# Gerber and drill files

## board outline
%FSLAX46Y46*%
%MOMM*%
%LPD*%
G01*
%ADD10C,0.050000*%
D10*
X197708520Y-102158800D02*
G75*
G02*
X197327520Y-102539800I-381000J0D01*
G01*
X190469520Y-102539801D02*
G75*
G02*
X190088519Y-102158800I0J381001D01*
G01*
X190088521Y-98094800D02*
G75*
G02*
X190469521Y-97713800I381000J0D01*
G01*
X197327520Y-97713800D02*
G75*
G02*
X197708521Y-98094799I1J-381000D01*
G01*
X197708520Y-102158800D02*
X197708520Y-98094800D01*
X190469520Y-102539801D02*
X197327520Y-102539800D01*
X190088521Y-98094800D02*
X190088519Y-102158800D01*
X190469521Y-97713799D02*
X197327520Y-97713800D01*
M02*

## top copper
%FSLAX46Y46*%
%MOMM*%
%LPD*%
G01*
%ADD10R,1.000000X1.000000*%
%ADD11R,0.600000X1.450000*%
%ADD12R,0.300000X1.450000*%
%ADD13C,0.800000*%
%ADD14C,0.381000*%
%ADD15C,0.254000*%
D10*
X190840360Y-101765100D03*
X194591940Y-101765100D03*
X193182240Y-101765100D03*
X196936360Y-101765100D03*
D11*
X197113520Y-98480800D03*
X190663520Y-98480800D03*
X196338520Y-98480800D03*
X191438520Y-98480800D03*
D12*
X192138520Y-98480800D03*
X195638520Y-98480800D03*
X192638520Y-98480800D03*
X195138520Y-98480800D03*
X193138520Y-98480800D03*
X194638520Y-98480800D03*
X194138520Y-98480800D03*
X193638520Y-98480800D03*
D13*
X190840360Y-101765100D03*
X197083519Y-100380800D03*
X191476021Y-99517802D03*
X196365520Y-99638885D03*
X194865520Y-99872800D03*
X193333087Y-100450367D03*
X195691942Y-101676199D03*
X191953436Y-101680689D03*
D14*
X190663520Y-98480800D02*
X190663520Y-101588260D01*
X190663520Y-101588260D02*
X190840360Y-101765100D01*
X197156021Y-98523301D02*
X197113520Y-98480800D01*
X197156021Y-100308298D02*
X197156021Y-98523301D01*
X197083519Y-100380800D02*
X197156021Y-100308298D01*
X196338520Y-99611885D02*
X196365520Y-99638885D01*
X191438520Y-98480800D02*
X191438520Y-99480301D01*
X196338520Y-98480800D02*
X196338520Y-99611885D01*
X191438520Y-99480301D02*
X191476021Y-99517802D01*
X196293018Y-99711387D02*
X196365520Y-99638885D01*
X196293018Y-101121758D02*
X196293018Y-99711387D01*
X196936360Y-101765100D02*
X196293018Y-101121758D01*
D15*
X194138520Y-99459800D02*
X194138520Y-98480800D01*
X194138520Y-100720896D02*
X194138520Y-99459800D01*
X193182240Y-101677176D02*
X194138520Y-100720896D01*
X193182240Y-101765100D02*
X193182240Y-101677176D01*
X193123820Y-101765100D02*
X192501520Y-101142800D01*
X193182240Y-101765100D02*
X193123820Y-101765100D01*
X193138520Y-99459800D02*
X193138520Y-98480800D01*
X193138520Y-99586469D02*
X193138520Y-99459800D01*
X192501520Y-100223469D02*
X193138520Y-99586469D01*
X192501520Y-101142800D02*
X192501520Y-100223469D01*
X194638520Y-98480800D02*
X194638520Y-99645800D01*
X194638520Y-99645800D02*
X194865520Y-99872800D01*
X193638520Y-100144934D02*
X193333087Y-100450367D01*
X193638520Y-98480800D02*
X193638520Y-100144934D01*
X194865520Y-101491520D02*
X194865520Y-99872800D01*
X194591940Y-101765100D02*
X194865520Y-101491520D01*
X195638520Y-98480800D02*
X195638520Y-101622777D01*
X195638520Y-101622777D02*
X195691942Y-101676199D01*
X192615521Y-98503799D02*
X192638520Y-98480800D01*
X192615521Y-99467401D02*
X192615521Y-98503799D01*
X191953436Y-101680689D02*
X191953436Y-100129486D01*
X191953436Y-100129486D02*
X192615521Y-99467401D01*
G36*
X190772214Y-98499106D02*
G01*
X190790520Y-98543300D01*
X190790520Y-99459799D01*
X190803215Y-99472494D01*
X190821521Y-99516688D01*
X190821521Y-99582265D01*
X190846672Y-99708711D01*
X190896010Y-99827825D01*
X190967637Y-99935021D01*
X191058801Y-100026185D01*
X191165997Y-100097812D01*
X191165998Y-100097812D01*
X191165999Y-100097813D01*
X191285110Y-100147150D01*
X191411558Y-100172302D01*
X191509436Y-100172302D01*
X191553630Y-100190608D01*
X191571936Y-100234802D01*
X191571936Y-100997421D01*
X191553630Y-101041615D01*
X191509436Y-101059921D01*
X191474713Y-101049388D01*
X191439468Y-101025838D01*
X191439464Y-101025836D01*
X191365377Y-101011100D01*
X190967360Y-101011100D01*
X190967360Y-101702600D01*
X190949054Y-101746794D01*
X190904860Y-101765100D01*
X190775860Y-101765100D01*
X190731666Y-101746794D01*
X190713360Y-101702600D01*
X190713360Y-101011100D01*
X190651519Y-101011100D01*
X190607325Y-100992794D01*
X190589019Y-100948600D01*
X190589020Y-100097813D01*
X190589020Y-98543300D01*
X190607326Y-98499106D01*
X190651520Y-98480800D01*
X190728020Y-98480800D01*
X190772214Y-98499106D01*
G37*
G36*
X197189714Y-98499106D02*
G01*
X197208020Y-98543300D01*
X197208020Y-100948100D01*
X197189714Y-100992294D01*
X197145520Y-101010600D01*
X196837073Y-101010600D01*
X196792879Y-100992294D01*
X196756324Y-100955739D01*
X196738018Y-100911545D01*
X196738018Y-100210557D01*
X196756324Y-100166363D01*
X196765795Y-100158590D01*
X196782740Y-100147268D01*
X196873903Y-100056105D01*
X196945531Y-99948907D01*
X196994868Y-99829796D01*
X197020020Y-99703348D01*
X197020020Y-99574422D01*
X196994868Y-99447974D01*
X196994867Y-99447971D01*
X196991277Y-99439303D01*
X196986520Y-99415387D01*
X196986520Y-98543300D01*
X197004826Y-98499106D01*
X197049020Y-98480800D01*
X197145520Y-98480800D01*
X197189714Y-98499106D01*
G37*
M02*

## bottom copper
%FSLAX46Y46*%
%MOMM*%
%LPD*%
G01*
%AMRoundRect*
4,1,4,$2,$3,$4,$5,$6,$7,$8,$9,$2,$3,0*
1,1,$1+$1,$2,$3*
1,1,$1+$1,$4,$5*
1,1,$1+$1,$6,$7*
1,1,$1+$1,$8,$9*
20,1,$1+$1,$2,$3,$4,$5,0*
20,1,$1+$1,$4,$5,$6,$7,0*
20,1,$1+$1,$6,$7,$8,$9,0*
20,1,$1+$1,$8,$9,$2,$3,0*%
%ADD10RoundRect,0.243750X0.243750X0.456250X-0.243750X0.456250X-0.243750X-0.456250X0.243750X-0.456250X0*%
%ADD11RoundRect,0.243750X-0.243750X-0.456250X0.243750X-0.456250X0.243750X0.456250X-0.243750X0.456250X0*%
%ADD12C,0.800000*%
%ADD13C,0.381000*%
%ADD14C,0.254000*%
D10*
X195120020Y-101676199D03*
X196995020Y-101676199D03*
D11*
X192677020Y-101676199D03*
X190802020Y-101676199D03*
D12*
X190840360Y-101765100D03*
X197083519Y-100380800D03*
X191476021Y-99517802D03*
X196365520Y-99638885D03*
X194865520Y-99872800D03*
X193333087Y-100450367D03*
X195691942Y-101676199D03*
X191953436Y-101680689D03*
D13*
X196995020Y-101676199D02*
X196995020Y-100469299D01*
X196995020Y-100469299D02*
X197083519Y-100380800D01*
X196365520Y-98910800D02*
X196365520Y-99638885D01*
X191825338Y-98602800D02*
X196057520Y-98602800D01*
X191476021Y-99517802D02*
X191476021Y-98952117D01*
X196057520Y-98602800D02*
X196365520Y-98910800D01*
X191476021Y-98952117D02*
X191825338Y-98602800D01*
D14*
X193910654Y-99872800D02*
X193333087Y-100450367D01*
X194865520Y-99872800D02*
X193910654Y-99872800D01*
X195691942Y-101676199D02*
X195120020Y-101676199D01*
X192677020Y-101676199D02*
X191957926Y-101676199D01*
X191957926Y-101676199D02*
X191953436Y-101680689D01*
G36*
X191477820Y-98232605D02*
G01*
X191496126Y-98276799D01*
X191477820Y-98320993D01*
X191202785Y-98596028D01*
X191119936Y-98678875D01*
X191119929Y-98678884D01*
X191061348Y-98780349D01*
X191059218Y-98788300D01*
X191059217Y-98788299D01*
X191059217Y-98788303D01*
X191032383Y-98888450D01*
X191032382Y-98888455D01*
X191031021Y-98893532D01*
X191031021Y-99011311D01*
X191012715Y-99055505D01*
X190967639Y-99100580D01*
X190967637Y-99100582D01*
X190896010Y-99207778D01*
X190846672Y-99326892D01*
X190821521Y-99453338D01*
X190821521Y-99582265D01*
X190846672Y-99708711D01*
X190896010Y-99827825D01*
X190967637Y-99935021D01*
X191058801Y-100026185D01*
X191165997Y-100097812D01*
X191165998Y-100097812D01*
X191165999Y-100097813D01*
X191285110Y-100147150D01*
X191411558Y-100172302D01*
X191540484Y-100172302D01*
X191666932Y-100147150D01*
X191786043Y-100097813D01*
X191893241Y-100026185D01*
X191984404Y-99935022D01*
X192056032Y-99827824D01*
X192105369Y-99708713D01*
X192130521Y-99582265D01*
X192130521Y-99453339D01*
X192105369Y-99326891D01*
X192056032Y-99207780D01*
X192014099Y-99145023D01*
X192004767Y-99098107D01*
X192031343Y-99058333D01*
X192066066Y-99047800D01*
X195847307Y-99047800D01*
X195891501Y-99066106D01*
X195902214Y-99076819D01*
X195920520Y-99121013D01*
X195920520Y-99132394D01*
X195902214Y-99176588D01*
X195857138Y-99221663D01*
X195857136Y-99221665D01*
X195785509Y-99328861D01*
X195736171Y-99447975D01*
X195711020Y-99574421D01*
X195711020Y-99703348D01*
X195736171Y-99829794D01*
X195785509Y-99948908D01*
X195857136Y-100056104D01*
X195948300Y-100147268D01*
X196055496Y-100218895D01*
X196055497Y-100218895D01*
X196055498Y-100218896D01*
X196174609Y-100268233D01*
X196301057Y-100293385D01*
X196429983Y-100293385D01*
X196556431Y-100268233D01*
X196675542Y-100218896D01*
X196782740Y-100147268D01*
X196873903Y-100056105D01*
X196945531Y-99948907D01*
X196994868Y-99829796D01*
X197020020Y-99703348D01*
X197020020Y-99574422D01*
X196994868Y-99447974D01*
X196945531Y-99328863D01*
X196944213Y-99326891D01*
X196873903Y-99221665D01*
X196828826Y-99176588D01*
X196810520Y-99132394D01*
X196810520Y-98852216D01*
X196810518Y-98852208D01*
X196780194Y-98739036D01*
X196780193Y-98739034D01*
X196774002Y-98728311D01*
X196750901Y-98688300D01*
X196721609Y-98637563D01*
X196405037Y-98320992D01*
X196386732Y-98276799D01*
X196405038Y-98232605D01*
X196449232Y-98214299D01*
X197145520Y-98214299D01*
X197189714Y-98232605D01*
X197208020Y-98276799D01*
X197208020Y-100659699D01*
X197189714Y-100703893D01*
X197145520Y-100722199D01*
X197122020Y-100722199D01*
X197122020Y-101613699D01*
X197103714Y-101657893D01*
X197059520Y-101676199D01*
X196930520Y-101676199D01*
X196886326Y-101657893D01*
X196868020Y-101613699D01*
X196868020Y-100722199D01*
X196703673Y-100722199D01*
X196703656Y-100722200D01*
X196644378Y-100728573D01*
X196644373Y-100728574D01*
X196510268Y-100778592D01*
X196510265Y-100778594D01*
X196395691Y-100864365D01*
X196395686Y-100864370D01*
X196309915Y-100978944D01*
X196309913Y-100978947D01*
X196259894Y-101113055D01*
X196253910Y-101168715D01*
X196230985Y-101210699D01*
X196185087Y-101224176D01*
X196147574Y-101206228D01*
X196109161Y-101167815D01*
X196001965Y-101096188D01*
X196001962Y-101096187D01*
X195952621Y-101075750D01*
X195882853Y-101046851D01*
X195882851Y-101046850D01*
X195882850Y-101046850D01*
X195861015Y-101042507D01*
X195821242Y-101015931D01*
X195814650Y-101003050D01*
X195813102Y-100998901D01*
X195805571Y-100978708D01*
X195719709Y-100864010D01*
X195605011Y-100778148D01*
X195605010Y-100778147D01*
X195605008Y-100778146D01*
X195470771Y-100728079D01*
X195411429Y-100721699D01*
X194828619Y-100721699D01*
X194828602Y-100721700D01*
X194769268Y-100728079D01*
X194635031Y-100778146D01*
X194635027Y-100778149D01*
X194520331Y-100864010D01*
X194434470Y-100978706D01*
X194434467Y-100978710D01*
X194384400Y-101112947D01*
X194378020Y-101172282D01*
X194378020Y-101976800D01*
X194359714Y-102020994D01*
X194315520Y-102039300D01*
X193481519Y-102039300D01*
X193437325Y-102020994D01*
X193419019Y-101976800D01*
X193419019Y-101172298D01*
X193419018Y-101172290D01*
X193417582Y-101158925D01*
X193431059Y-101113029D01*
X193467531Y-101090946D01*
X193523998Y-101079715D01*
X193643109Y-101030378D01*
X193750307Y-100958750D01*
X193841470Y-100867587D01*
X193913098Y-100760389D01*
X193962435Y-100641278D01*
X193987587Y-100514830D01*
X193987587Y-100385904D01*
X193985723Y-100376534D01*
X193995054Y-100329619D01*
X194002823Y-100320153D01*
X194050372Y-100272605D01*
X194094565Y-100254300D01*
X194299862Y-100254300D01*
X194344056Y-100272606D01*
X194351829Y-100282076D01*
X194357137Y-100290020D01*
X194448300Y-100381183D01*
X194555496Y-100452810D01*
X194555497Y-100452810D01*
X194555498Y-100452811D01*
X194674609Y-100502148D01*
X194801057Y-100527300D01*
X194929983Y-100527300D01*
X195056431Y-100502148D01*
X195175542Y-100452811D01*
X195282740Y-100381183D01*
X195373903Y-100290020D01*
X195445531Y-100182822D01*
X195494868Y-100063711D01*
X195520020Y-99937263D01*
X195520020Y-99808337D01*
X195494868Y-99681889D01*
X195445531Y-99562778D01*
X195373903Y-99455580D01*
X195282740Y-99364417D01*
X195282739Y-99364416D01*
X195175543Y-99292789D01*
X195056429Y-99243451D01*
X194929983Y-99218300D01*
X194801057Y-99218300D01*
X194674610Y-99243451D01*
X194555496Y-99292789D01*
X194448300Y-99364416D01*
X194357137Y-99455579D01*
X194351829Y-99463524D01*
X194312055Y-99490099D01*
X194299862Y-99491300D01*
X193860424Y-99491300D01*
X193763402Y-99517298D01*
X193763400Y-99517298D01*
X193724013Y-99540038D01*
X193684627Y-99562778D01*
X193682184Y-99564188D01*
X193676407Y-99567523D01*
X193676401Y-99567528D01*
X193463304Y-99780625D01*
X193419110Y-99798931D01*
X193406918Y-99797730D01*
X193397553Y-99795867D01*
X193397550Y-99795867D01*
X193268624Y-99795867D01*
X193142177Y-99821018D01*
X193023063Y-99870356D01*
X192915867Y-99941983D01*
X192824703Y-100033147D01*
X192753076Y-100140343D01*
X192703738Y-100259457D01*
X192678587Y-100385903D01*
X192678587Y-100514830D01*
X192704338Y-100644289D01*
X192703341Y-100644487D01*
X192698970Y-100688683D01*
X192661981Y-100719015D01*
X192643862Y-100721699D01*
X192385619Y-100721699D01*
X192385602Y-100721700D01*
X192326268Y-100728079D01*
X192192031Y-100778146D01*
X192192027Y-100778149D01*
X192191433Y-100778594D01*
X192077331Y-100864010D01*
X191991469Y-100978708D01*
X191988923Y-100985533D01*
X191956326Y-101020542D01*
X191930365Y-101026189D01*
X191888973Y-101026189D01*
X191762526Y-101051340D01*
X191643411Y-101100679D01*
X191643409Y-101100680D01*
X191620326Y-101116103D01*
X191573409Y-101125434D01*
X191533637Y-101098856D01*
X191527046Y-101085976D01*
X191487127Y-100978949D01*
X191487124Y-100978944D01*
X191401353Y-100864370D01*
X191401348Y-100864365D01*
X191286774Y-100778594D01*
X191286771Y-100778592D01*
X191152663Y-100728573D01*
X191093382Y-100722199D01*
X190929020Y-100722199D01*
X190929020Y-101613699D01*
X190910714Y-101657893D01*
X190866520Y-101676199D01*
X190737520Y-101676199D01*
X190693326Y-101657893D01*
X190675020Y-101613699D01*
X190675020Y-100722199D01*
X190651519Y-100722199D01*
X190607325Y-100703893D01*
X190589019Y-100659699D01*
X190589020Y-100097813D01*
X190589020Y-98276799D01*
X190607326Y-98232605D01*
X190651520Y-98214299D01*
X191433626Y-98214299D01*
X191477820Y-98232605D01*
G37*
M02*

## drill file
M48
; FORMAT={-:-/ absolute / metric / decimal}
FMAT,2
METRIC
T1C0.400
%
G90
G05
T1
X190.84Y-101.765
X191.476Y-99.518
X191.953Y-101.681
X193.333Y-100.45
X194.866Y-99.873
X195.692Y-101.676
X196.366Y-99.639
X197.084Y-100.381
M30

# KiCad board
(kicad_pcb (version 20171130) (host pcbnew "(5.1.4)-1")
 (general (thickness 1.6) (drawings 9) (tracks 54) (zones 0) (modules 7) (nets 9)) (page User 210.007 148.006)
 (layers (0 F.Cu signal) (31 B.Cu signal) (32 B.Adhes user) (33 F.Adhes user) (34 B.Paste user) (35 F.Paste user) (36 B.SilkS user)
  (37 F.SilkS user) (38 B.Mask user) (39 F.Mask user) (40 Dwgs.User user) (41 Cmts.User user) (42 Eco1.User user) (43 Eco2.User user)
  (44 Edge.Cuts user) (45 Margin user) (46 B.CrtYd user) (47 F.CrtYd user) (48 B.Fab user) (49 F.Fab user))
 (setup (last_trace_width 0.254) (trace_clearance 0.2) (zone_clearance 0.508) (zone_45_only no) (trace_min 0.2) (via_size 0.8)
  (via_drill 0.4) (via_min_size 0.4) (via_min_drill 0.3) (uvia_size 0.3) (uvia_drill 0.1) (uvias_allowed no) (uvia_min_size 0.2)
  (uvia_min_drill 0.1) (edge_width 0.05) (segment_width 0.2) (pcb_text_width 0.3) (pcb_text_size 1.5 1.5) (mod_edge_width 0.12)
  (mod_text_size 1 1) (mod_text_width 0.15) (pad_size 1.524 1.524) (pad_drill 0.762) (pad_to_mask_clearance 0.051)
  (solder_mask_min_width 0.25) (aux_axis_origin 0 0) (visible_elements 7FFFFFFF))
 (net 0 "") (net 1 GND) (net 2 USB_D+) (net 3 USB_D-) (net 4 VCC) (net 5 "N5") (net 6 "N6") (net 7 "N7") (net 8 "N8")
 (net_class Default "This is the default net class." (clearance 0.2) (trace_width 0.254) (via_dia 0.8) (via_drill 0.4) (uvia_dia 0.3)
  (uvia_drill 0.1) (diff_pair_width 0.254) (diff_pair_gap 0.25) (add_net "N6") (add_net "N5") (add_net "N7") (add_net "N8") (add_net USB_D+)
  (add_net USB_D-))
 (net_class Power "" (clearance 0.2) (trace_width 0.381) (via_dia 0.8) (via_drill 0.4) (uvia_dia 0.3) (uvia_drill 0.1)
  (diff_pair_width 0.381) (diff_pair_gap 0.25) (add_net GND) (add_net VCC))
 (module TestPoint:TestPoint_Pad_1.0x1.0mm (layer F.Cu) (at 190.84036 101.7651 180)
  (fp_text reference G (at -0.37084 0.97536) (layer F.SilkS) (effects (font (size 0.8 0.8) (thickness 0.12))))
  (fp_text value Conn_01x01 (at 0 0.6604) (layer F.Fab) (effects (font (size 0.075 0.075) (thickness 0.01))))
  (pad 1 smd rect (at 0 0 180) (size 1 1) (layers F.Cu F.Mask) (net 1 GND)))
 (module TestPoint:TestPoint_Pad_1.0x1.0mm (layer F.Cu) (at 194.59194 101.7651 270)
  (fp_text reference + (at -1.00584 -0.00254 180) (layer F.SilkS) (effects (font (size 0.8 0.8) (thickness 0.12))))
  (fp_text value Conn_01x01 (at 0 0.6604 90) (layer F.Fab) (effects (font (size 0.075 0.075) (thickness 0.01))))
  (pad 1 smd rect (at 0 0 270) (size 1 1) (layers F.Cu F.Mask) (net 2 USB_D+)))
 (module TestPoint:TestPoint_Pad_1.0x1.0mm (layer F.Cu) (at 193.18224 101.7651 270)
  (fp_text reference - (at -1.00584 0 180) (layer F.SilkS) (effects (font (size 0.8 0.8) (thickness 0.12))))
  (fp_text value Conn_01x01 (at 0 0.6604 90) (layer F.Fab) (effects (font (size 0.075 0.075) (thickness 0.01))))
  (pad 1 smd rect (at 0 0 270) (size 1 1) (layers F.Cu F.Mask) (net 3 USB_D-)))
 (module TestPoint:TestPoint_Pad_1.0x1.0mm (layer F.Cu) (at 196.93636 101.7651 180)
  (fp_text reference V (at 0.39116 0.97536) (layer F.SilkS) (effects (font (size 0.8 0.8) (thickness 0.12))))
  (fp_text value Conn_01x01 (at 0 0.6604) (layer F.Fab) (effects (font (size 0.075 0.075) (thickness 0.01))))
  (pad 1 smd rect (at 0 0 180) (size 1 1) (layers F.Cu F.Mask) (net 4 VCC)))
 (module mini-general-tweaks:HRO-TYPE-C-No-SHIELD (layer F.Cu) (at 193.89852 98.4758)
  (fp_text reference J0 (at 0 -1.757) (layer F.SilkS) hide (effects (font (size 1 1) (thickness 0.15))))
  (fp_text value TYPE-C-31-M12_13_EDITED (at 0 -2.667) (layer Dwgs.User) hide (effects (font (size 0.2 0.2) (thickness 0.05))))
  (pad 12 smd rect (at 3.215 0.005) (size 0.6 1.45) (layers F.Cu F.Paste F.Mask) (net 1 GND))
  (pad 1 smd rect (at -3.235 0.005) (size 0.6 1.45) (layers F.Cu F.Paste F.Mask) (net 1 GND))
  (pad 11 smd rect (at 2.44 0.005) (size 0.6 1.45) (layers F.Cu F.Paste F.Mask) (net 4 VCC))
  (pad 2 smd rect (at -2.46 0.005) (size 0.6 1.45) (layers F.Cu F.Paste F.Mask) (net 4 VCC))
  (pad 3 smd rect (at -1.76 0.005) (size 0.3 1.45) (layers F.Cu F.Paste F.Mask) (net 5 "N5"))
  (pad 10 smd rect (at 1.74 0.005) (size 0.3 1.45) (layers F.Cu F.Paste F.Mask) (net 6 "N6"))
  (pad 4 smd rect (at -1.26 0.005) (size 0.3 1.45) (layers F.Cu F.Paste F.Mask) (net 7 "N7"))
  (pad 9 smd rect (at 1.24 0.005) (size 0.3 1.45) (layers F.Cu F.Paste F.Mask) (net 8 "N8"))
  (pad 5 smd rect (at -0.76 0.005) (size 0.3 1.45) (layers F.Cu F.Paste F.Mask) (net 3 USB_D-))
  (pad 8 smd rect (at 0.74 0.005) (size 0.3 1.45) (layers F.Cu F.Paste F.Mask) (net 2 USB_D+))
  (pad 7 smd rect (at 0.24 0.005) (size 0.3 1.45) (layers F.Cu F.Paste F.Mask) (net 3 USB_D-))
  (pad 6 smd rect (at -0.26 0.005) (size 0.3 1.45) (layers F.Cu F.Paste F.Mask) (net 2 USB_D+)))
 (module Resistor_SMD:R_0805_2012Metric (layer B.Cu) (at 196.05752 101.676199 180)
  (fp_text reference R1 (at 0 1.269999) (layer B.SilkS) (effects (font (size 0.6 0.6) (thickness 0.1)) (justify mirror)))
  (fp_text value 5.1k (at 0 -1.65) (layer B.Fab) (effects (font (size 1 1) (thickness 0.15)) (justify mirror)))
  (pad 2 smd roundrect (at 0.9375 0 180) (size 0.975 1.4) (layers B.Cu B.Paste B.Mask) (roundrect_rratio 0.25) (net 6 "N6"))
  (pad 1 smd roundrect (at -0.9375 0 180) (size 0.975 1.4) (layers B.Cu B.Paste B.Mask) (roundrect_rratio 0.25) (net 1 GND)))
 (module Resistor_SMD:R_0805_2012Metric (layer B.Cu) (at 191.73952 101.676199)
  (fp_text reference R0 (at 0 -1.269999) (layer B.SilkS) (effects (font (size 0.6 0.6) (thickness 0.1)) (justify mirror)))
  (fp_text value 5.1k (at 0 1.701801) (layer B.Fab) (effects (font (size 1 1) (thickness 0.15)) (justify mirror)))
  (pad 2 smd roundrect (at 0.9375 0) (size 0.975 1.4) (layers B.Cu B.Paste B.Mask) (roundrect_rratio 0.25) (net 7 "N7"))
  (pad 1 smd roundrect (at -0.9375 0) (size 0.975 1.4) (layers B.Cu B.Paste B.Mask) (roundrect_rratio 0.25) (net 1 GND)))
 (gr_arc (start 197.32752 102.1588) (end 197.70852 102.1588) (angle 90) (layer Edge.Cuts) (width 0.05))
 (gr_arc (start 190.46952 102.1588) (end 190.46952 102.539801) (angle 90) (layer Edge.Cuts) (width 0.05))
 (gr_arc (start 190.469521 98.0948) (end 190.088521 98.0948) (angle 90) (layer Edge.Cuts) (width 0.05))
 (gr_arc (start 197.327521 98.0948) (end 197.32752 97.7138) (angle 90) (layer Edge.Cuts) (width 0.05))
 (gr_line (start 197.70852 102.1588) (end 197.70852 98.0948) (layer Edge.Cuts) (width 0.05))
 (gr_line (start 190.46952 102.539801) (end 197.32752 102.5398) (layer Edge.Cuts) (width 0.05))
 (gr_line (start 190.088521 98.0948) (end 190.088519 102.1588) (layer Edge.Cuts) (width 0.05))
 (gr_line (start 190.469521 97.713799) (end 197.32752 97.7138) (layer Edge.Cuts) (width 0.05))
 (via (at 190.84036 101.7651) (size 0.8) (drill 0.4) (layers F.Cu B.Cu) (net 1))
 (segment (start 190.66352 98.4808) (end 190.66352 101.58826) (width 0.381) (layer F.Cu) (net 1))
 (segment (start 190.66352 101.58826) (end 190.84036 101.7651) (width 0.381) (layer F.Cu) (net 1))
 (segment (start 196.99502 101.676199) (end 196.99502 100.469299) (width 0.381) (layer B.Cu) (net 1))
 (segment (start 197.156021 98.523301) (end 197.11352 98.4808) (width 0.381) (layer F.Cu) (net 1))
 (segment (start 197.156021 100.308298) (end 197.156021 98.523301) (width 0.381) (layer F.Cu) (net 1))
 (segment (start 197.083519 100.3808) (end 197.156021 100.308298) (width 0.381) (layer F.Cu) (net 1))
 (segment (start 196.99502 100.469299) (end 197.083519 100.3808) (width 0.381) (layer B.Cu) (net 1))
 (via (at 197.083519 100.3808) (size 0.8) (drill 0.4) (layers F.Cu B.Cu) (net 1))
 (via (at 191.476021 99.517802) (size 0.8) (drill 0.4) (layers F.Cu B.Cu) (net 4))
 (via (at 196.36552 99.638885) (size 0.8) (drill 0.4) (layers F.Cu B.Cu) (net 4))
 (segment (start 196.36552 98.9108) (end 196.36552 99.638885) (width 0.381) (layer B.Cu) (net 4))
 (segment (start 196.33852 99.611885) (end 196.36552 99.638885) (width 0.381) (layer F.Cu) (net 4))
 (segment (start 191.825338 98.6028) (end 196.05752 98.6028) (width 0.381) (layer B.Cu) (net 4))
 (segment (start 191.476021 99.517802) (end 191.476021 98.952117) (width 0.381) (layer B.Cu) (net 4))
 (segment (start 196.05752 98.6028) (end 196.36552 98.9108) (width 0.381) (layer B.Cu) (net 4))
 (segment (start 191.476021 98.952117) (end 191.825338 98.6028) (width 0.381) (layer B.Cu) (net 4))
 (segment (start 191.43852 98.4808) (end 191.43852 99.480301) (width 0.381) (layer F.Cu) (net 4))
 (segment (start 196.33852 98.4808) (end 196.33852 99.611885) (width 0.381) (layer F.Cu) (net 4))
 (segment (start 191.43852 99.480301) (end 191.476021 99.517802) (width 0.381) (layer F.Cu) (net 4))
 (segment (start 196.293018 99.711387) (end 196.36552 99.638885) (width 0.381) (layer F.Cu) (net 4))
 (segment (start 196.293018 101.121758) (end 196.293018 99.711387) (width 0.381) (layer F.Cu) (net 4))
 (segment (start 196.93636 101.7651) (end 196.293018 101.121758) (width 0.381) (layer F.Cu) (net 4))
 (segment (start 194.13852 99.4598) (end 194.13852 98.4808) (width 0.254) (layer F.Cu) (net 3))
 (segment (start 194.13852 100.720896) (end 194.13852 99.4598) (width 0.254) (layer F.Cu) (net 3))
 (segment (start 193.18224 101.677176) (end 194.13852 100.720896) (width 0.254) (layer F.Cu) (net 3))
 (segment (start 193.18224 101.7651) (end 193.18224 101.677176) (width 0.254) (layer F.Cu) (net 3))
 (segment (start 193.12382 101.7651) (end 192.50152 101.1428) (width 0.254) (layer F.Cu) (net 3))
 (segment (start 193.18224 101.7651) (end 193.12382 101.7651) (width 0.254) (layer F.Cu) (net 3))
 (segment (start 193.13852 99.4598) (end 193.13852 98.4808) (width 0.254) (layer F.Cu) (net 3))
 (segment (start 193.13852 99.586469) (end 193.13852 99.4598) (width 0.254) (layer F.Cu) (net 3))
 (segment (start 192.50152 100.223469) (end 193.13852 99.586469) (width 0.254) (layer F.Cu) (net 3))
 (segment (start 192.50152 101.1428) (end 192.50152 100.223469) (width 0.254) (layer F.Cu) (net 3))
 (segment (start 194.63852 98.4808) (end 194.63852 99.6458) (width 0.254) (layer F.Cu) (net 2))
 (segment (start 194.63852 99.6458) (end 194.86552 99.8728) (width 0.254) (layer F.Cu) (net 2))
 (via (at 194.86552 99.8728) (size 0.8) (drill 0.4) (layers F.Cu B.Cu) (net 2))
 (via (at 193.333087 100.450367) (size 0.8) (drill 0.4) (layers F.Cu B.Cu) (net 2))
 (segment (start 193.910654 99.8728) (end 193.333087 100.450367) (width 0.254) (layer B.Cu) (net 2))
 (segment (start 193.63852 100.144934) (end 193.333087 100.450367) (width 0.254) (layer F.Cu) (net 2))
 (segment (start 193.63852 98.4808) (end 193.63852 100.144934) (width 0.254) (layer F.Cu) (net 2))
 (segment (start 194.86552 99.8728) (end 193.910654 99.8728) (width 0.254) (layer B.Cu) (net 2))
 (segment (start 194.86552 101.49152) (end 194.86552 99.8728) (width 0.254) (layer F.Cu) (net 2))
 (segment (start 194.59194 101.7651) (end 194.86552 101.49152) (width 0.254) (layer F.Cu) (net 2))
 (via (at 195.691942 101.676199) (size 0.8) (drill 0.4) (layers F.Cu B.Cu) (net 6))
 (segment (start 195.63852 98.4808) (end 195.63852 101.622777) (width 0.254) (layer F.Cu) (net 6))
 (segment (start 195.63852 101.622777) (end 195.691942 101.676199) (width 0.254) (layer F.Cu) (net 6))
 (segment (start 195.691942 101.676199) (end 195.12002 101.676199) (width 0.254) (layer B.Cu) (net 6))
 (via (at 191.953436 101.680689) (size 0.8) (drill 0.4) (layers F.Cu B.Cu) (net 7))
 (segment (start 192.67702 101.676199) (end 191.957926 101.676199) (width 0.254) (layer B.Cu) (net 7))
 (segment (start 191.957926 101.676199) (end 191.953436 101.680689) (width 0.254) (layer B.Cu) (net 7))
 (segment (start 192.615521 98.503799) (end 192.63852 98.4808) (width 0.254) (layer F.Cu) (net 7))
 (segment (start 192.615521 99.467401) (end 192.615521 98.503799) (width 0.254) (layer F.Cu) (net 7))
 (segment (start 191.953436 101.680689) (end 191.953436 100.129486) (width 0.254) (layer F.Cu) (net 7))
 (segment (start 191.953436 100.129486) (end 192.615521 99.467401) (width 0.254) (layer F.Cu) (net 7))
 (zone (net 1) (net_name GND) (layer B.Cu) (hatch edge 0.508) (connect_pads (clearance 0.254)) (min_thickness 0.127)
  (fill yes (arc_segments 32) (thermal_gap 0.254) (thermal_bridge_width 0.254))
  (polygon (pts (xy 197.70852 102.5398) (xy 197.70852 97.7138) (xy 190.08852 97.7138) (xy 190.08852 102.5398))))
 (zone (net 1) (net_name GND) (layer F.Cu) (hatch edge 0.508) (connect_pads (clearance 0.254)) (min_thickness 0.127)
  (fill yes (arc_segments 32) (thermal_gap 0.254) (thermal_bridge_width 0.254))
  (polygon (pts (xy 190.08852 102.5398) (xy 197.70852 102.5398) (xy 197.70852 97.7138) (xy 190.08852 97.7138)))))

